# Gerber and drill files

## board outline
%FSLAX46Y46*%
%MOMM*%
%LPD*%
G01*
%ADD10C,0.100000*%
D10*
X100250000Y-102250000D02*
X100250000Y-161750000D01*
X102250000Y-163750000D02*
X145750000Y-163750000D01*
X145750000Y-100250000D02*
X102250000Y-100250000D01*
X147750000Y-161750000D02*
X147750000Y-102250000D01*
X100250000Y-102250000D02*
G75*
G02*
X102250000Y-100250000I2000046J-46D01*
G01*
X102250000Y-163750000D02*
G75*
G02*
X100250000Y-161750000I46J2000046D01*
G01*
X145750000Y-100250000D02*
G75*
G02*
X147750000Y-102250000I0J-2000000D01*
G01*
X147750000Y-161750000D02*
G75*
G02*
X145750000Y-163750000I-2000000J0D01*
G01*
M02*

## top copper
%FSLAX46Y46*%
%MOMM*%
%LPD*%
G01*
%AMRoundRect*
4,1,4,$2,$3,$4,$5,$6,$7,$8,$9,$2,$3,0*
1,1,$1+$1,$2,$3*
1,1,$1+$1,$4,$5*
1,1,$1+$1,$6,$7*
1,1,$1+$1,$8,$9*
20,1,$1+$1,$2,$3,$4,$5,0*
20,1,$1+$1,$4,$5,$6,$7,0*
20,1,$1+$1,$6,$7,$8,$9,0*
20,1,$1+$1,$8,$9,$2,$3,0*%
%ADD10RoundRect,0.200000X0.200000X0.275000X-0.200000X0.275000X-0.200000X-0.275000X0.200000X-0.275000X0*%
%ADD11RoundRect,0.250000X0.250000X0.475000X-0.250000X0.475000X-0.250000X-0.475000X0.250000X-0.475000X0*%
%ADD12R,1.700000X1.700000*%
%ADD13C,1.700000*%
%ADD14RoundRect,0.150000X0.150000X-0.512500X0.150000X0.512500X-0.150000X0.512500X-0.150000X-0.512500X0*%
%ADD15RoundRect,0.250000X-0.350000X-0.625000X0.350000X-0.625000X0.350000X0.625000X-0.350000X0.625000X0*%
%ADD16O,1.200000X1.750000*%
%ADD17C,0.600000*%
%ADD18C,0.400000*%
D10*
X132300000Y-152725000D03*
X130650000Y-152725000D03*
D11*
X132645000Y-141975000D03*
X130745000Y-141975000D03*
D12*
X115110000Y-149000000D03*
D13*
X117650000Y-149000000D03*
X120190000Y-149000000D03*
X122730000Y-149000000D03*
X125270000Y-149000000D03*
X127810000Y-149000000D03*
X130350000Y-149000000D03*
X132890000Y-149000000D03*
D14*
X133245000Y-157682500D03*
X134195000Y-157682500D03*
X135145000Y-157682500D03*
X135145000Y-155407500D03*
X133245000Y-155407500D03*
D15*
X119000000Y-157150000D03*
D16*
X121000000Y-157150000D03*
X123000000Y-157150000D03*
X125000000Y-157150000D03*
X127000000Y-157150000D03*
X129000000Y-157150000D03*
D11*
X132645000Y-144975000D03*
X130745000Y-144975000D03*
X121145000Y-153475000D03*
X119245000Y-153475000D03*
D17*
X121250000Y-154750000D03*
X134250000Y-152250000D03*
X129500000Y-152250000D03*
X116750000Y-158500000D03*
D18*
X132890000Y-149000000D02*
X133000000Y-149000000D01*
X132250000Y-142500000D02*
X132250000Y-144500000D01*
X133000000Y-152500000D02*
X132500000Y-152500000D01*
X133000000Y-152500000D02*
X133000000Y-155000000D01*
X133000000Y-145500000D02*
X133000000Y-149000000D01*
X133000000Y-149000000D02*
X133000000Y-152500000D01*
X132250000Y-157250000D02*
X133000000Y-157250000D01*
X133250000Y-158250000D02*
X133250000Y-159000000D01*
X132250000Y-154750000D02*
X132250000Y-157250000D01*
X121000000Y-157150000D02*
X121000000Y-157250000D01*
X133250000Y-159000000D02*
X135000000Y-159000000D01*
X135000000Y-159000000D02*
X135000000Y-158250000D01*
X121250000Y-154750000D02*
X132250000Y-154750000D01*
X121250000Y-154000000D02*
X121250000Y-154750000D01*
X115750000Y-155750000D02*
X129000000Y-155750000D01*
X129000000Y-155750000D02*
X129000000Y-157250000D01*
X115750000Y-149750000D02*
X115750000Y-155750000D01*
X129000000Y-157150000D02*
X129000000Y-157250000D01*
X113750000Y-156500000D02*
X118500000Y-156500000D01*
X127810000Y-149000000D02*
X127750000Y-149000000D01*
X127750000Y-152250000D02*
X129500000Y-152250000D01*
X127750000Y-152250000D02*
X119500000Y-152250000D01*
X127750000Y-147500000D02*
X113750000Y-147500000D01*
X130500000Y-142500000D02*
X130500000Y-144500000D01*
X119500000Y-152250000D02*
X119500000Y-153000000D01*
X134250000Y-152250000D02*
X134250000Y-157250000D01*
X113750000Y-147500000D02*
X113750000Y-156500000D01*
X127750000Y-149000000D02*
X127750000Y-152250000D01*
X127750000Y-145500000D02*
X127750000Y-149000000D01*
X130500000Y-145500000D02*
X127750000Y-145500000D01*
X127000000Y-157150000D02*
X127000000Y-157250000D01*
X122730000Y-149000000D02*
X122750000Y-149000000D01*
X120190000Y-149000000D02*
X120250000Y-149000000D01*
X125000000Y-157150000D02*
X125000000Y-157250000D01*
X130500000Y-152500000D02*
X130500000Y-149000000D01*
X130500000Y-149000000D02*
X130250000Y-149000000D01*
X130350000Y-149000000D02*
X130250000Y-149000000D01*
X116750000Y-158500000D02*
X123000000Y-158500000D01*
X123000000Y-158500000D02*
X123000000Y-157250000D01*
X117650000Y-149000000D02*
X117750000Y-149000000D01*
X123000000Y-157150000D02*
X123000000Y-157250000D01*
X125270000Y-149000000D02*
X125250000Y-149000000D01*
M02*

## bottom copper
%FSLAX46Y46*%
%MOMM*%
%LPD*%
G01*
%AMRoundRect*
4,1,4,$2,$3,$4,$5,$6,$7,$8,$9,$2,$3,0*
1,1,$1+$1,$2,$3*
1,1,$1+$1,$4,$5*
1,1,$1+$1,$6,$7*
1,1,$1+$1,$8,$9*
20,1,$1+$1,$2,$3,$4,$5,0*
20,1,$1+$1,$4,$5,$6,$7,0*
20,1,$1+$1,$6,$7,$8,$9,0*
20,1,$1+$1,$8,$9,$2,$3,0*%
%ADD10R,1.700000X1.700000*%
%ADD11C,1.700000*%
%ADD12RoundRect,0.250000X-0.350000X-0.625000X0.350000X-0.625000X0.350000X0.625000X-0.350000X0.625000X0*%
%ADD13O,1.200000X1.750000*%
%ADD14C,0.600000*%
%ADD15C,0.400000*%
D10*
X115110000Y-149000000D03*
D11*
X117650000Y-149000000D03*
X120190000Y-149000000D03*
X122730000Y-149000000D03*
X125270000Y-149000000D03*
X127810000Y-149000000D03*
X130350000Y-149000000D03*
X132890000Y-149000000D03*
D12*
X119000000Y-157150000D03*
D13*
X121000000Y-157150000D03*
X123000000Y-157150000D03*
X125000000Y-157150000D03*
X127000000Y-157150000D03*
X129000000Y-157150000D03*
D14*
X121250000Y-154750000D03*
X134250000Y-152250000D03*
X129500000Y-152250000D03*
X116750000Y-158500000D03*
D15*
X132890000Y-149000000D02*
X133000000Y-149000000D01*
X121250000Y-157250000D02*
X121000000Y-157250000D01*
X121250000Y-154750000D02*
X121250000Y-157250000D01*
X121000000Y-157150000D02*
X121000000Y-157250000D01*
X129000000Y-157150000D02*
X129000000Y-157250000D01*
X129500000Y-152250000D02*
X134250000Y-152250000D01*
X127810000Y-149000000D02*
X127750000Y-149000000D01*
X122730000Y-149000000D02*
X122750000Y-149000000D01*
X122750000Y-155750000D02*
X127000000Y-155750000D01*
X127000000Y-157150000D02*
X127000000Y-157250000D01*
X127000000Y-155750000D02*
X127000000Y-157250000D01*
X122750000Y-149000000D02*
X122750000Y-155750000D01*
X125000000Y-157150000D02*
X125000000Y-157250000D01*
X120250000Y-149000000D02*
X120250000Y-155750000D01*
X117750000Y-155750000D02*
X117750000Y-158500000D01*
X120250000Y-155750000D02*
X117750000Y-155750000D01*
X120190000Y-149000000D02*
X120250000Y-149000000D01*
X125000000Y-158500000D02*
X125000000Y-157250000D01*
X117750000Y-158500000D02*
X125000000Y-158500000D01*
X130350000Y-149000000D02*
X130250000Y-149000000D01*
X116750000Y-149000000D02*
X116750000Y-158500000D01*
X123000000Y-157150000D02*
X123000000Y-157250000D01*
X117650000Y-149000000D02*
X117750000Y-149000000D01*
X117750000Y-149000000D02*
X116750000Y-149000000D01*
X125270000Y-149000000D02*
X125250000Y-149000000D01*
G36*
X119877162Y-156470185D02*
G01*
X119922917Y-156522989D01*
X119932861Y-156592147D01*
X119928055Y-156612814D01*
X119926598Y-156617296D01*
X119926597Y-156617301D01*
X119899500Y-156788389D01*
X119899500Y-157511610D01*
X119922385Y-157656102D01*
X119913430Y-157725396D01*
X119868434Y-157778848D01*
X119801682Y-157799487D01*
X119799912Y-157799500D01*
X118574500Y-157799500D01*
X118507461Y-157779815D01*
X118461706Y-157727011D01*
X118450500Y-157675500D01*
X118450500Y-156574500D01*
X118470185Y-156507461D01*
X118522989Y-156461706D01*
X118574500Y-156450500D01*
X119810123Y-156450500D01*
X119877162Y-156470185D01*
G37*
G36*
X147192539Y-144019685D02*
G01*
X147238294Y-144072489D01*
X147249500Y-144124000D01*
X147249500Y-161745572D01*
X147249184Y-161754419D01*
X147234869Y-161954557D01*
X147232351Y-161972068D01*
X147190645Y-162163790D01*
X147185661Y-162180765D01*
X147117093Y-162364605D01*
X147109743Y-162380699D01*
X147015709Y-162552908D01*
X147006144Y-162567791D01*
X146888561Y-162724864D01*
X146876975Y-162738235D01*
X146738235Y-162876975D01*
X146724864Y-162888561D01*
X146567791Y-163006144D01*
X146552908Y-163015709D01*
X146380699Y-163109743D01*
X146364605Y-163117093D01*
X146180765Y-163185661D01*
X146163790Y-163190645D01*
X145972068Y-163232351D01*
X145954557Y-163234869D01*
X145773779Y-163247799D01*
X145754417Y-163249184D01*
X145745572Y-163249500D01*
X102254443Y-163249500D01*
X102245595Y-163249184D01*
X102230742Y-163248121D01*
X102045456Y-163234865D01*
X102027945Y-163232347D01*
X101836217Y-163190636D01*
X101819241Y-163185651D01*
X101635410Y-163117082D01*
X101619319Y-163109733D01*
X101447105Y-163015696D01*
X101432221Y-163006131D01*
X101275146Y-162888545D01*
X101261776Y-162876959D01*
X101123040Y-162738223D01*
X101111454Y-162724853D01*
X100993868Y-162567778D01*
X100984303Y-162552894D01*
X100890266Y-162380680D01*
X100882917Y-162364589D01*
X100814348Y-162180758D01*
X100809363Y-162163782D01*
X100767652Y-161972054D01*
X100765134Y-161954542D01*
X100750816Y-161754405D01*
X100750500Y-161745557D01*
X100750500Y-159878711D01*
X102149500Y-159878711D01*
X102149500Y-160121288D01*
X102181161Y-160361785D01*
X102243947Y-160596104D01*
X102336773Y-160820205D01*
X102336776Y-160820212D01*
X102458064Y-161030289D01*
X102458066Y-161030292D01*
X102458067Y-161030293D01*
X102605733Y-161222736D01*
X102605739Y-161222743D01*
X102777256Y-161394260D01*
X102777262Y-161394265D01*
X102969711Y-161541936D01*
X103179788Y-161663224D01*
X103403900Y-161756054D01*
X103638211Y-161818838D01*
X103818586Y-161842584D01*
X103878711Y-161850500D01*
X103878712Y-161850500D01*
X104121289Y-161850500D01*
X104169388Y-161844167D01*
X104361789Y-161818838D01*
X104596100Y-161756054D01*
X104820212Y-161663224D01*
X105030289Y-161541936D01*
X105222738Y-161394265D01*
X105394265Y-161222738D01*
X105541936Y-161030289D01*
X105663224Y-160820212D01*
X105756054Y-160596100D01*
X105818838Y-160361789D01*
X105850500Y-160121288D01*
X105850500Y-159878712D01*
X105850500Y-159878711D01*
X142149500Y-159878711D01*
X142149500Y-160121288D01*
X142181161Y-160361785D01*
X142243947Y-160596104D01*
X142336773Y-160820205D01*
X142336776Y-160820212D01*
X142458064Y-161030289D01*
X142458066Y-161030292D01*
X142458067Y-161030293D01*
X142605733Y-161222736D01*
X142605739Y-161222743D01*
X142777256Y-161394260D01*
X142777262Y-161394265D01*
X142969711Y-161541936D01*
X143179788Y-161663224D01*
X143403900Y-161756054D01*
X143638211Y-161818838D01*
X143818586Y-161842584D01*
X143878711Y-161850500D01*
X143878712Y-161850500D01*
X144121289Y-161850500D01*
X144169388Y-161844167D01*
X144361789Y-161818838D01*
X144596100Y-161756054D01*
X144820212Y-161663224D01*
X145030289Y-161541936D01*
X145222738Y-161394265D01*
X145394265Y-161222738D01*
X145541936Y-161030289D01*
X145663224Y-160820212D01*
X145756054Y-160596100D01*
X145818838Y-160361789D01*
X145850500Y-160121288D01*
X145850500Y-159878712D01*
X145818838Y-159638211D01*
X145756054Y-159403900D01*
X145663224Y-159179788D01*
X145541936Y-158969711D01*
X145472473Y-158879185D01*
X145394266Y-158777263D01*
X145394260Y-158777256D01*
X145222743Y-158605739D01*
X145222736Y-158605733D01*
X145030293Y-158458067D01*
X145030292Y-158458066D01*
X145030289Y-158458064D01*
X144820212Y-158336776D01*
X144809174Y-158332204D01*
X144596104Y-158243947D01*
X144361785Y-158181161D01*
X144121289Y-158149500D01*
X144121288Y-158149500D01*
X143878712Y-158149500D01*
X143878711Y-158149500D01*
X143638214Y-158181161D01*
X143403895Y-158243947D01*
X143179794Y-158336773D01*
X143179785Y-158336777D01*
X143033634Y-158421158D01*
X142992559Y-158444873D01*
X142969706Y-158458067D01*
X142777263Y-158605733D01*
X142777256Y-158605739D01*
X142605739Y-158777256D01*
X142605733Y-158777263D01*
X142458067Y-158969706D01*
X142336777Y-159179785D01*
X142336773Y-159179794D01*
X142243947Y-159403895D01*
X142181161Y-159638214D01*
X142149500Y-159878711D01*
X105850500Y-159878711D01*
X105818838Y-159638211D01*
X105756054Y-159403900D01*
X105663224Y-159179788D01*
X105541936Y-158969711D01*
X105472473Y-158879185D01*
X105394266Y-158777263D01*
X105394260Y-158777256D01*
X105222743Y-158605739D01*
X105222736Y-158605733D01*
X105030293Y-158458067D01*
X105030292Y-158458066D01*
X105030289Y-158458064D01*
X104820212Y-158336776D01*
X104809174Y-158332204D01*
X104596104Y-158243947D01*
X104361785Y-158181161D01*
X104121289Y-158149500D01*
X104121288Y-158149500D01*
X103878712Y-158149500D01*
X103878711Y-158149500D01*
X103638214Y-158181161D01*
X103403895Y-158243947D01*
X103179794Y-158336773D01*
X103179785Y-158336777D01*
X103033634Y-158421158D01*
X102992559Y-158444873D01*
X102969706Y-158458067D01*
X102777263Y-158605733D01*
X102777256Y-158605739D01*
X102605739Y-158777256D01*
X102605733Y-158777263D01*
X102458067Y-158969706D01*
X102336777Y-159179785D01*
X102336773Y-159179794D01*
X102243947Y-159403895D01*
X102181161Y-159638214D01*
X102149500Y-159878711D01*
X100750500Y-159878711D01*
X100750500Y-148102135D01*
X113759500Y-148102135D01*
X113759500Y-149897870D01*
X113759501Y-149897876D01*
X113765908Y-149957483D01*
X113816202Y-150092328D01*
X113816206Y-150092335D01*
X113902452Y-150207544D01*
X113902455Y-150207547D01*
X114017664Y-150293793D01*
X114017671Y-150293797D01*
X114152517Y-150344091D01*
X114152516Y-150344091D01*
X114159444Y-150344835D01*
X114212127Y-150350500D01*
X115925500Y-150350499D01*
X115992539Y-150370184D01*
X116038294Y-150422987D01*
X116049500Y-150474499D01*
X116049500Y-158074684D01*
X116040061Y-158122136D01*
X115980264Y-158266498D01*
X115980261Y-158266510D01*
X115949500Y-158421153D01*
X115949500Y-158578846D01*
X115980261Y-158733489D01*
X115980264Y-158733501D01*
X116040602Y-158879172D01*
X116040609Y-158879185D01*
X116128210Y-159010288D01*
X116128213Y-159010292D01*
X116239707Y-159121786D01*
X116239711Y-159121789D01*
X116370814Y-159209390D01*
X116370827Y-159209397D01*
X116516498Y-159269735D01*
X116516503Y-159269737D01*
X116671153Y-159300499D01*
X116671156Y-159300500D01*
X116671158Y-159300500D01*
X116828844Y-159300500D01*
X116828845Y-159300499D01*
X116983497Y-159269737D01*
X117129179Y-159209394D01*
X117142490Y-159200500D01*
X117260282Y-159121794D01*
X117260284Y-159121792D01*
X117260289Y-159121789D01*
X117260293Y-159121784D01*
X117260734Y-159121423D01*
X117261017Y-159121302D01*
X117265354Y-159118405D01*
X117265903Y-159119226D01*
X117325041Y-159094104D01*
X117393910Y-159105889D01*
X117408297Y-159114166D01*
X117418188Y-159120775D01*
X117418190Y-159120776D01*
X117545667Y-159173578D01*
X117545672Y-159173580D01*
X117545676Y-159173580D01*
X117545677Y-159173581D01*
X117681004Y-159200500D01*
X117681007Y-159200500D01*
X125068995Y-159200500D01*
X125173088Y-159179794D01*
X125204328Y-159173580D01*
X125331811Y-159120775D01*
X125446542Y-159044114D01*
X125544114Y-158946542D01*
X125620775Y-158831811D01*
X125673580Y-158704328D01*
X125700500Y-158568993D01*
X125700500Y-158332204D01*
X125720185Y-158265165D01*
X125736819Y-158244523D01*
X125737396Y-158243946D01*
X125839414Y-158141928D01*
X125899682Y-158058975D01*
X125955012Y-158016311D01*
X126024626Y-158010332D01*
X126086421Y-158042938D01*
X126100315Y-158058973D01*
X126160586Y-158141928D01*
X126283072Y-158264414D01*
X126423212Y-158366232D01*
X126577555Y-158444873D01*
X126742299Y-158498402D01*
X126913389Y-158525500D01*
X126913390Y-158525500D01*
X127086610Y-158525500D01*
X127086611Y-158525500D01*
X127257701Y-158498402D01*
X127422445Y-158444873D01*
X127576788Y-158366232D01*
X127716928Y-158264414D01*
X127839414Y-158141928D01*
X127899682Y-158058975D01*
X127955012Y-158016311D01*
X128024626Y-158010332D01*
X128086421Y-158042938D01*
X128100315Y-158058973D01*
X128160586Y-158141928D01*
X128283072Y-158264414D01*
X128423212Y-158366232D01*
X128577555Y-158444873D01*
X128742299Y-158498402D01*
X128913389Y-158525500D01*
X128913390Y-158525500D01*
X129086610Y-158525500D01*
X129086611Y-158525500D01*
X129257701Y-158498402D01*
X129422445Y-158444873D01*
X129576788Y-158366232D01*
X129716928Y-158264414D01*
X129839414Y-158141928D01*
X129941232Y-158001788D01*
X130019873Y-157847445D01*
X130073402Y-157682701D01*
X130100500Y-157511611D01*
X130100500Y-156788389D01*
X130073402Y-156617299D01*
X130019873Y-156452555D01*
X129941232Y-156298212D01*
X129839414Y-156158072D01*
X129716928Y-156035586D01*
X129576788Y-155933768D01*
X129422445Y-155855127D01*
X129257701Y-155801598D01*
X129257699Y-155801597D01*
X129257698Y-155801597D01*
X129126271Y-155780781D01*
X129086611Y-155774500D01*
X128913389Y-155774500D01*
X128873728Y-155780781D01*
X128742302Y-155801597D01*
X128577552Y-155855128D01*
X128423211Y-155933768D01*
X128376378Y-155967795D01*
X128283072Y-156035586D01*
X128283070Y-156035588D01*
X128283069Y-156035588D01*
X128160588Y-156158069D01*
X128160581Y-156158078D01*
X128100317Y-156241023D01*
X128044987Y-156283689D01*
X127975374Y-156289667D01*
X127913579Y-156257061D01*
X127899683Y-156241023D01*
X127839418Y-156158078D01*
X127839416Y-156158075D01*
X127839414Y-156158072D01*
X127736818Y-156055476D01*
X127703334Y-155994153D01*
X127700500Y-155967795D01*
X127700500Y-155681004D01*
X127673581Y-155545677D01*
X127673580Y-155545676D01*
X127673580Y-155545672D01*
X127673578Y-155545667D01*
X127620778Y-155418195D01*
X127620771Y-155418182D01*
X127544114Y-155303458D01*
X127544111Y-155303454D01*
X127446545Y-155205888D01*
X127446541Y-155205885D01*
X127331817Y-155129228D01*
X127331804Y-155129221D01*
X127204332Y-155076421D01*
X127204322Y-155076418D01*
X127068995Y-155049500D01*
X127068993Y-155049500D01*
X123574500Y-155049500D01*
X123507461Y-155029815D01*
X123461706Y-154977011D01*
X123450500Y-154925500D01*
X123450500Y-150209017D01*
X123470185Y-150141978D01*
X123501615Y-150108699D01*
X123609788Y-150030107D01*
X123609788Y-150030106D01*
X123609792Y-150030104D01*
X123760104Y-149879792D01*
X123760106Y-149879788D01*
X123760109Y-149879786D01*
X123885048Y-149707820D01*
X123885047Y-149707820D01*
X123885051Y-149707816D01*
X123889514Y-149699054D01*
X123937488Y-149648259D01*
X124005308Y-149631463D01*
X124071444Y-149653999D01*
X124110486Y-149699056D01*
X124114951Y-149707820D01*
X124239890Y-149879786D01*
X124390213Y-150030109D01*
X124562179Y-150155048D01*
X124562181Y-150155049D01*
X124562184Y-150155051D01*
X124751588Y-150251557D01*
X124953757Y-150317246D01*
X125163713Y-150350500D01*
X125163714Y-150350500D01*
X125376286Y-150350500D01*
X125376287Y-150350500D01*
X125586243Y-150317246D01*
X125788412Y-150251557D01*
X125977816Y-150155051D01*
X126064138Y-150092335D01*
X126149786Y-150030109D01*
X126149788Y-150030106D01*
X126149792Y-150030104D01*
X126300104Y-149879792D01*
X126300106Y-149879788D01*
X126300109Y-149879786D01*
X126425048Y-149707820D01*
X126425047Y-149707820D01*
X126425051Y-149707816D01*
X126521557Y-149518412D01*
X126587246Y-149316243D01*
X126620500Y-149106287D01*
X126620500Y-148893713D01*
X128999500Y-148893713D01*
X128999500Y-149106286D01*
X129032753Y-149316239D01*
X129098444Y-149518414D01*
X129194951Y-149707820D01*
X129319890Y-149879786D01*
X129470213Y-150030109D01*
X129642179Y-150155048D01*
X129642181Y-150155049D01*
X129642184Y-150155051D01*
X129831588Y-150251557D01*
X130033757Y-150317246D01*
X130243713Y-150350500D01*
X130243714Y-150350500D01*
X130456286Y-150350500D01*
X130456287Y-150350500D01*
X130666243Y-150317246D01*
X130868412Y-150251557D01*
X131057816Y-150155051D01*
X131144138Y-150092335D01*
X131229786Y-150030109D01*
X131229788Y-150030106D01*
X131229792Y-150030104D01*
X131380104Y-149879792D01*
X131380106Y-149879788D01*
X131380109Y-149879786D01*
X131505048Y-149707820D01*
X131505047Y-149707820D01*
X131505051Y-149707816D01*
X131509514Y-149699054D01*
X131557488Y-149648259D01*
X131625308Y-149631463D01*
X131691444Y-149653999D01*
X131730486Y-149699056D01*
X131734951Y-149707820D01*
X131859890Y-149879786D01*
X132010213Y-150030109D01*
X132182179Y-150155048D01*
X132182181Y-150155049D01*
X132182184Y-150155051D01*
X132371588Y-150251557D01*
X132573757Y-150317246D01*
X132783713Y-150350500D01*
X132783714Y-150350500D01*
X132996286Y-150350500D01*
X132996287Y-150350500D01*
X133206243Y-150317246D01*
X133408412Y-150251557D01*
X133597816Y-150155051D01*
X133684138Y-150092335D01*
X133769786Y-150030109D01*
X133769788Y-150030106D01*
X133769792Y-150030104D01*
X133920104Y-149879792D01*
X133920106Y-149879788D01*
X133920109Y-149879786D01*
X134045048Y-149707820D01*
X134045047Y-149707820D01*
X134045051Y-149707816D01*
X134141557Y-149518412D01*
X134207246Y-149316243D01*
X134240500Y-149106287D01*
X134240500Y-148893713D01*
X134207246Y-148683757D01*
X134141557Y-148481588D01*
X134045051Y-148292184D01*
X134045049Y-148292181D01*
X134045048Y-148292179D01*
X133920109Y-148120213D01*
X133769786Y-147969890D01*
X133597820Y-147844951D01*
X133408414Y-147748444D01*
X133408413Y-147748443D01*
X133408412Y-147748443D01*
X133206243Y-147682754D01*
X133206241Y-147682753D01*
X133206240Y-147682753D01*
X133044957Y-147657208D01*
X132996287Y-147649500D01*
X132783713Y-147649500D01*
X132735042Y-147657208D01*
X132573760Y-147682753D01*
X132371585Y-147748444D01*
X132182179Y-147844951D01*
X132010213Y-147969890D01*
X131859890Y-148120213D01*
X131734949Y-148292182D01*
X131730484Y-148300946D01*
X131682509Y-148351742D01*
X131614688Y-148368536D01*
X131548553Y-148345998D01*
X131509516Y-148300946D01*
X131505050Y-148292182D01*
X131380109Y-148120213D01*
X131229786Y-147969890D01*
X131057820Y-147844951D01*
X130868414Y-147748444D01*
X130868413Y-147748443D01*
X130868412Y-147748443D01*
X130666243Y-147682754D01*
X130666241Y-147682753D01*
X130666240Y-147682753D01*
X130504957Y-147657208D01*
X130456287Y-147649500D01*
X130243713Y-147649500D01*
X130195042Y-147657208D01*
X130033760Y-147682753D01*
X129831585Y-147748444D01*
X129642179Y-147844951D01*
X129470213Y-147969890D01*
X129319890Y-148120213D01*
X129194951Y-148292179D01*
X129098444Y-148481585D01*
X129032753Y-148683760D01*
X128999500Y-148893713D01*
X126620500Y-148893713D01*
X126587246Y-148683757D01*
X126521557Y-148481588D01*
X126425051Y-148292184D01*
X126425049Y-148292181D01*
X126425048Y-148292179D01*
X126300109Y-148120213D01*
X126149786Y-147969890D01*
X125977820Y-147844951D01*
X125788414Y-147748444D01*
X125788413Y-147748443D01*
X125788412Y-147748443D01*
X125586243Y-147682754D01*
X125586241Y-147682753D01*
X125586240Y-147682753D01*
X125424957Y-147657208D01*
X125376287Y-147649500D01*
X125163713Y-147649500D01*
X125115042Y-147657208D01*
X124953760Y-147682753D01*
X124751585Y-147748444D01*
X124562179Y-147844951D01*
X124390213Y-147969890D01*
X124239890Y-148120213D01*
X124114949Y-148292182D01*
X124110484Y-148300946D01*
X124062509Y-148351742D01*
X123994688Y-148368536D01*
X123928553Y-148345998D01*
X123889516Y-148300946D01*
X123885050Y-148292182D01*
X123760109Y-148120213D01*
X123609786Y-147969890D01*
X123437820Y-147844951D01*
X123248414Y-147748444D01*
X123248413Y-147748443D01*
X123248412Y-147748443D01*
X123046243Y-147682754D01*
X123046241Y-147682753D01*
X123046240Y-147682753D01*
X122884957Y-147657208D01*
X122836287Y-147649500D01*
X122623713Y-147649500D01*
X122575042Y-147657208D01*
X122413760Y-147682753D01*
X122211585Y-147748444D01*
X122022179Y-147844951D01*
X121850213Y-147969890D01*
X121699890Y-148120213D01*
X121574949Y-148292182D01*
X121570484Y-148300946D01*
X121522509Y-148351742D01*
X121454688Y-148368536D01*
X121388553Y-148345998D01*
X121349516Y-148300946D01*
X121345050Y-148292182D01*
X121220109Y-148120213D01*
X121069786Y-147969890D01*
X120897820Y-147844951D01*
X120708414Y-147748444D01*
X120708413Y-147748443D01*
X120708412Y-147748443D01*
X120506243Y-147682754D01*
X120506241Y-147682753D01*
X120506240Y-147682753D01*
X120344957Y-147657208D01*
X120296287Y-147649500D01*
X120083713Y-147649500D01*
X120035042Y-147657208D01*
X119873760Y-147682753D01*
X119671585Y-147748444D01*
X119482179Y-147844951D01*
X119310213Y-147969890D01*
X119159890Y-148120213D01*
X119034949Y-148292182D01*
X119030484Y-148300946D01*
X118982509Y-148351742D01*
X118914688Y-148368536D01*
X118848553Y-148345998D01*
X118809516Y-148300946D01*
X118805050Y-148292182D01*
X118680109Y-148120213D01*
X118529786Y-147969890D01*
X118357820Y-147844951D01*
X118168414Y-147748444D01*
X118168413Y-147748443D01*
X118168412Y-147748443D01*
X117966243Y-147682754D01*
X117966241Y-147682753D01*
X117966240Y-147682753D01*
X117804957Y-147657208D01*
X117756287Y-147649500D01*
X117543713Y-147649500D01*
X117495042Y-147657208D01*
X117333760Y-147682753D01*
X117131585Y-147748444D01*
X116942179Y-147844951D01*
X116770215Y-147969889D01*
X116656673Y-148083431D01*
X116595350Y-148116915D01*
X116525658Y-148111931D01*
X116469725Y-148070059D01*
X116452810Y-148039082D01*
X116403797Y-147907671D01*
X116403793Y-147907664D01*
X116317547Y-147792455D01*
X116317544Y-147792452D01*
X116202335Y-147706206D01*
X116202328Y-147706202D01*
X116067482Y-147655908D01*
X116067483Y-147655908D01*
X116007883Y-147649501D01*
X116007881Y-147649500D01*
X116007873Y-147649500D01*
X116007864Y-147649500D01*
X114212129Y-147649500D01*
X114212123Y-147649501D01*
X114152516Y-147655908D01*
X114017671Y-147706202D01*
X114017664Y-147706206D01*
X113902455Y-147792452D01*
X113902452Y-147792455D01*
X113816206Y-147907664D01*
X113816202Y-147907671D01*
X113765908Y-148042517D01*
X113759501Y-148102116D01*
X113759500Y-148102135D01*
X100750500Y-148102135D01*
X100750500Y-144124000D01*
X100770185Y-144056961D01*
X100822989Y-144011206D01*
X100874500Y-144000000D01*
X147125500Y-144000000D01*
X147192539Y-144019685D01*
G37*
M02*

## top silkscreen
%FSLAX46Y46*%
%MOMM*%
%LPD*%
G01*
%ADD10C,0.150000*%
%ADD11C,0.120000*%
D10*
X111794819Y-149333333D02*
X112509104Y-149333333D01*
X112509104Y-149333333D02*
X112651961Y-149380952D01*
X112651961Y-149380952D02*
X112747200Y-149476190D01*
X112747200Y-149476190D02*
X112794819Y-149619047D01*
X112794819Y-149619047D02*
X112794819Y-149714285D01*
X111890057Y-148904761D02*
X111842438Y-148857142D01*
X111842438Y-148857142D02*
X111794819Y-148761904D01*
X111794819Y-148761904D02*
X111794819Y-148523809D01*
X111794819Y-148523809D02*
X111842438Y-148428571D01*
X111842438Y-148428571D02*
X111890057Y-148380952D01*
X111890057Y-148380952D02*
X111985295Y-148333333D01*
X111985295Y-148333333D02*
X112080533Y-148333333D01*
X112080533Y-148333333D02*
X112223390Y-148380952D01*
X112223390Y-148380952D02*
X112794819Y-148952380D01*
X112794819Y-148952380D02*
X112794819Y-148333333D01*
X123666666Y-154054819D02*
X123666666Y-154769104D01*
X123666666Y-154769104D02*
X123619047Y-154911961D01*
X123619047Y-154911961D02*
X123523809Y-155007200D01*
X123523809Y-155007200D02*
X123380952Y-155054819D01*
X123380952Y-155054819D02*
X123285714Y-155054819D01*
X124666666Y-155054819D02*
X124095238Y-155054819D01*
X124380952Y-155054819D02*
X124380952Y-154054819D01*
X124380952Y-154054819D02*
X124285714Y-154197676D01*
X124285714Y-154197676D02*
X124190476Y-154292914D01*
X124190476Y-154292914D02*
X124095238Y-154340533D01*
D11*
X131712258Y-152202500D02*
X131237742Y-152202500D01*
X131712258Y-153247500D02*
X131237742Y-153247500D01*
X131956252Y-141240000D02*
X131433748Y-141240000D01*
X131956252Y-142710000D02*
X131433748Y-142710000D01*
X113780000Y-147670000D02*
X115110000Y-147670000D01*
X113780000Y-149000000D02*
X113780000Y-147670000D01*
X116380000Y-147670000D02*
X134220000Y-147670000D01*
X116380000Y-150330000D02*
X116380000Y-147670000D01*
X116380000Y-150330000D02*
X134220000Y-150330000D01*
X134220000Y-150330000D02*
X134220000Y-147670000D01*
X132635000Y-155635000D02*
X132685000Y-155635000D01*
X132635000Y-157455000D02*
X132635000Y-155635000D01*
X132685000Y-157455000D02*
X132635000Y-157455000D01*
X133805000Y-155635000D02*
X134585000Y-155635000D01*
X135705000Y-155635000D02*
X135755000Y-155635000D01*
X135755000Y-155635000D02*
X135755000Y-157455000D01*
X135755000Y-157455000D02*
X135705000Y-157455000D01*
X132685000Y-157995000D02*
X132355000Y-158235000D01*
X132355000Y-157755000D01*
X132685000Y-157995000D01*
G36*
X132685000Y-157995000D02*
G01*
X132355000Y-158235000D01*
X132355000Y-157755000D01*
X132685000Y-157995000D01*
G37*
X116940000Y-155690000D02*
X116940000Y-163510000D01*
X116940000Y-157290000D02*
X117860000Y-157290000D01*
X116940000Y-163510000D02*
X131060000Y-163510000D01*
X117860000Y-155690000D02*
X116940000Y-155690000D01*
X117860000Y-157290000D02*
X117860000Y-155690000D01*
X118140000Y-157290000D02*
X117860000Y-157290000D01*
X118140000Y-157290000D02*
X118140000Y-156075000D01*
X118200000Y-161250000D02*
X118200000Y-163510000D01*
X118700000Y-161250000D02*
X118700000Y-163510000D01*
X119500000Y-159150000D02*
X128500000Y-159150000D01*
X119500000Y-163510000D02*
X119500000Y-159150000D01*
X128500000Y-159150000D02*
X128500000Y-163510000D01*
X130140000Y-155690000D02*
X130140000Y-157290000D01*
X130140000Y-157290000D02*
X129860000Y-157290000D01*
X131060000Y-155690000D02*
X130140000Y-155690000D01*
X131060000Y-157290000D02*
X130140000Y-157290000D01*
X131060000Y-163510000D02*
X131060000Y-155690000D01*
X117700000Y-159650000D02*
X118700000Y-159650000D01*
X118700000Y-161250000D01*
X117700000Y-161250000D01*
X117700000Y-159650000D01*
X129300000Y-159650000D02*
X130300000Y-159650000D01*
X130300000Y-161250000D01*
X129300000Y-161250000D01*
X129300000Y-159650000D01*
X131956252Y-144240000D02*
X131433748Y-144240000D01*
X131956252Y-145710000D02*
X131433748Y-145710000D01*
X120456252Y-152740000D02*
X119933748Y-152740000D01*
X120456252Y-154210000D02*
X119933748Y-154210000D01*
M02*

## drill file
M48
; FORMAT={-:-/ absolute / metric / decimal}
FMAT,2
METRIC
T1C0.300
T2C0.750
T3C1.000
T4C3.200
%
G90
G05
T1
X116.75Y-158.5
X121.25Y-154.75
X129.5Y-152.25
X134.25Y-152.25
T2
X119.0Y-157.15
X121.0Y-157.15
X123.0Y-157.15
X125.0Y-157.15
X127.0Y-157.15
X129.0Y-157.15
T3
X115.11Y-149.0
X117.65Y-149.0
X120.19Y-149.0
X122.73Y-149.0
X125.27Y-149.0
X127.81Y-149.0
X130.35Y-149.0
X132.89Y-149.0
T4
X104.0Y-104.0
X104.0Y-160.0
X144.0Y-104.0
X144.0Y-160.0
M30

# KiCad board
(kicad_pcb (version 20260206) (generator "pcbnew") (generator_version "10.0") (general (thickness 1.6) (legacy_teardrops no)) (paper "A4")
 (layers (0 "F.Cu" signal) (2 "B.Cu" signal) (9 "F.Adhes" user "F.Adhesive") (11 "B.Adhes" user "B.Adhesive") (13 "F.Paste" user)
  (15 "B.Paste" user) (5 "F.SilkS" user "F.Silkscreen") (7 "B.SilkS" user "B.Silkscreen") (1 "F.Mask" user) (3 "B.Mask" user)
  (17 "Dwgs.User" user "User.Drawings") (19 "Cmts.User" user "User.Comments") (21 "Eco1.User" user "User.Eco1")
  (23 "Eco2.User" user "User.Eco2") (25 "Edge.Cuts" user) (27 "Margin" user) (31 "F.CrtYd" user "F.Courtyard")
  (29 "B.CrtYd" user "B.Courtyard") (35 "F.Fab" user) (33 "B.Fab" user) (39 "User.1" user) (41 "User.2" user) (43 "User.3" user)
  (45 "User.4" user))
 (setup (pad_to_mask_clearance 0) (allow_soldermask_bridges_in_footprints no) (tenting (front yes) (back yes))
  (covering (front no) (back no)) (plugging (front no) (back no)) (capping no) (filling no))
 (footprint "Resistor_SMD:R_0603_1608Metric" (layer "F.Cu") (at 131.475 152.725 180)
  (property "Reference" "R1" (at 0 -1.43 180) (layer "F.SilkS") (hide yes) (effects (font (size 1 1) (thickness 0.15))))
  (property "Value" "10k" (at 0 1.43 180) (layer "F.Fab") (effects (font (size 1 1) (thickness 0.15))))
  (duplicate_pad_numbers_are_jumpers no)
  (fp_line (start -0.237258 0.5225) (end 0.237258 0.5225) (stroke (width 0.12) (type solid)) (layer "F.SilkS"))
  (fp_line (start -0.237258 -0.5225) (end 0.237258 -0.5225) (stroke (width 0.12) (type solid)) (layer "F.SilkS"))
  (pad "1" smd roundrect (at -0.825 0 180) (size 0.8 0.95) (layers "F.Cu" "F.Mask" "F.Paste") (roundrect_rratio 0.25) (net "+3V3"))
  (pad "2" smd roundrect (at 0.825 0 180) (size 0.8 0.95) (layers "F.Cu" "F.Mask" "F.Paste") (roundrect_rratio 0.25) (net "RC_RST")))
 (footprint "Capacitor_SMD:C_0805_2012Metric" (layer "F.Cu") (at 131.695 141.975 180)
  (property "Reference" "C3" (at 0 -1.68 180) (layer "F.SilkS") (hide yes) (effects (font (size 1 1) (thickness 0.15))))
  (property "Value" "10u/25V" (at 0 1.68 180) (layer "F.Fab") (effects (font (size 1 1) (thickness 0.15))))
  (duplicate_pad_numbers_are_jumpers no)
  (fp_line (start -0.261252 0.735) (end 0.261252 0.735) (stroke (width 0.12) (type solid)) (layer "F.SilkS"))
  (fp_line (start -0.261252 -0.735) (end 0.261252 -0.735) (stroke (width 0.12) (type solid)) (layer "F.SilkS"))
  (pad "1" smd roundrect (at -0.95 0 180) (size 1 1.45) (layers "F.Cu" "F.Mask" "F.Paste") (roundrect_rratio 0.25) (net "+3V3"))
  (pad "2" smd roundrect (at 0.95 0 180) (size 1 1.45) (layers "F.Cu" "F.Mask" "F.Paste") (roundrect_rratio 0.25) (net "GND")))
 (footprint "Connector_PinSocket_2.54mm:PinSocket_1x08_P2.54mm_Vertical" (layer "F.Cu") (at 115.11 149 90)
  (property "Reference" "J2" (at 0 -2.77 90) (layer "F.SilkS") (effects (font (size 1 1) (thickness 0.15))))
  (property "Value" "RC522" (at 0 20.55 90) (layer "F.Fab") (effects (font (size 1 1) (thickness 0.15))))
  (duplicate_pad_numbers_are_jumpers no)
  (fp_line (start 1.33 -1.33) (end 1.33 0) (stroke (width 0.12) (type solid)) (layer "F.SilkS"))
  (fp_line (start 0 -1.33) (end 1.33 -1.33) (stroke (width 0.12) (type solid)) (layer "F.SilkS"))
  (fp_line (start 1.33 1.27) (end 1.33 19.11) (stroke (width 0.12) (type solid)) (layer "F.SilkS"))
  (fp_line (start -1.33 1.27) (end 1.33 1.27) (stroke (width 0.12) (type solid)) (layer "F.SilkS"))
  (fp_line (start -1.33 1.27) (end -1.33 19.11) (stroke (width 0.12) (type solid)) (layer "F.SilkS"))
  (fp_line (start -1.33 19.11) (end 1.33 19.11) (stroke (width 0.12) (type solid)) (layer "F.SilkS"))
  (pad "1" thru_hole rect (at 0 0 90) (size 1.7 1.7) (drill 1) (layers "*.Cu" "*.Mask") (remove_unused_layers no) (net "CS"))
  (pad "2" thru_hole circle (at 0 2.54 90) (size 1.7 1.7) (drill 1) (layers "*.Cu" "*.Mask") (remove_unused_layers no) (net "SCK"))
  (pad "3" thru_hole circle (at 0 5.08 90) (size 1.7 1.7) (drill 1) (layers "*.Cu" "*.Mask") (remove_unused_layers no) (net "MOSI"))
  (pad "4" thru_hole circle (at 0 7.62 90) (size 1.7 1.7) (drill 1) (layers "*.Cu" "*.Mask") (remove_unused_layers no) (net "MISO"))
  (pad "5" thru_hole circle (at 0 10.16 90) (size 1.7 1.7) (drill 1) (layers "*.Cu" "*.Mask") (remove_unused_layers no)
   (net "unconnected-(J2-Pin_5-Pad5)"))
  (pad "6" thru_hole circle (at 0 12.7 90) (size 1.7 1.7) (drill 1) (layers "*.Cu" "*.Mask") (remove_unused_layers no) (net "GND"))
  (pad "7" thru_hole circle (at 0 15.24 90) (size 1.7 1.7) (drill 1) (layers "*.Cu" "*.Mask") (remove_unused_layers no) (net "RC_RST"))
  (pad "8" thru_hole circle (at 0 17.78 90) (size 1.7 1.7) (drill 1) (layers "*.Cu" "*.Mask") (remove_unused_layers no) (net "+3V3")))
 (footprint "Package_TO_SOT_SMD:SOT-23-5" (layer "F.Cu") (at 134.195 156.545 90)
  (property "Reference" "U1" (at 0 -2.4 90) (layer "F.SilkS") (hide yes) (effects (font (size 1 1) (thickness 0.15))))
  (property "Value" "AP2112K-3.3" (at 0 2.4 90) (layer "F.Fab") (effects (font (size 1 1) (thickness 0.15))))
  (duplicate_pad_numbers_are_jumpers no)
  (fp_line (start 0.91 -1.56) (end 0.91 -1.51) (stroke (width 0.12) (type solid)) (layer "F.SilkS"))
  (fp_line (start -0.91 -1.56) (end 0.91 -1.56) (stroke (width 0.12) (type solid)) (layer "F.SilkS"))
  (fp_line (start -0.91 -1.51) (end -0.91 -1.56) (stroke (width 0.12) (type solid)) (layer "F.SilkS"))
  (fp_line (start 0.91 -0.39) (end 0.91 0.39) (stroke (width 0.12) (type solid)) (layer "F.SilkS"))
  (fp_line (start 0.91 1.51) (end 0.91 1.56) (stroke (width 0.12) (type solid)) (layer "F.SilkS"))
  (fp_line (start 0.91 1.56) (end -0.91 1.56) (stroke (width 0.12) (type solid)) (layer "F.SilkS"))
  (fp_line (start -0.91 1.56) (end -0.91 1.51) (stroke (width 0.12) (type solid)) (layer "F.SilkS"))
  (fp_poly (pts (xy -1.45 -1.51) (xy -1.69 -1.84) (xy -1.21 -1.84)) (stroke (width 0.12) (type solid)) (fill yes) (layer "F.SilkS"))
  (pad "1" smd roundrect (at -1.1375 -0.95 90) (size 1.325 0.6) (layers "F.Cu" "F.Mask" "F.Paste") (roundrect_rratio 0.25) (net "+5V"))
  (pad "2" smd roundrect (at -1.1375 0 90) (size 1.325 0.6) (layers "F.Cu" "F.Mask" "F.Paste") (roundrect_rratio 0.25) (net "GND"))
  (pad "3" smd roundrect (at -1.1375 0.95 90) (size 1.325 0.6) (layers "F.Cu" "F.Mask" "F.Paste") (roundrect_rratio 0.25) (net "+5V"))
  (pad "4" smd roundrect (at 1.1375 0.95 90) (size 1.325 0.6) (layers "F.Cu" "F.Mask" "F.Paste") (roundrect_rratio 0.25)
   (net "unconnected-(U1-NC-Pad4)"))
  (pad "5" smd roundrect (at 1.1375 -0.95 90) (size 1.325 0.6) (layers "F.Cu" "F.Mask" "F.Paste") (roundrect_rratio 0.25) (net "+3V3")))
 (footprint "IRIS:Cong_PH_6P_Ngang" (layer "F.Cu") (at 119 157.15)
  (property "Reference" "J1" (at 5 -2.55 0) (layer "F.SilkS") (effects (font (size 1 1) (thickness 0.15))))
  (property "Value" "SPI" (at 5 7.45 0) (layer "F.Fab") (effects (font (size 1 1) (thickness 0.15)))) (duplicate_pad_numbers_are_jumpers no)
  (fp_line (start -2.06 -1.46) (end -2.06 6.36) (stroke (width 0.12) (type solid)) (layer "F.SilkS"))
  (fp_line (start -2.06 0.14) (end -1.14 0.14) (stroke (width 0.12) (type solid)) (layer "F.SilkS"))
  (fp_line (start -2.06 6.36) (end 12.06 6.36) (stroke (width 0.12) (type solid)) (layer "F.SilkS"))
  (fp_line (start -1.14 -1.46) (end -2.06 -1.46) (stroke (width 0.12) (type solid)) (layer "F.SilkS"))
  (fp_line (start -1.14 0.14) (end -1.14 -1.46) (stroke (width 0.12) (type solid)) (layer "F.SilkS"))
  (fp_line (start -0.86 0.14) (end -1.14 0.14) (stroke (width 0.12) (type solid)) (layer "F.SilkS"))
  (fp_line (start -0.86 0.14) (end -0.86 -1.075) (stroke (width 0.12) (type solid)) (layer "F.SilkS"))
  (fp_line (start -0.8 4.1) (end -0.8 6.36) (stroke (width 0.12) (type solid)) (layer "F.SilkS"))
  (fp_line (start -0.3 4.1) (end -0.3 6.36) (stroke (width 0.12) (type solid)) (layer "F.SilkS"))
  (fp_line (start 0.5 2) (end 9.5 2) (stroke (width 0.12) (type solid)) (layer "F.SilkS"))
  (fp_line (start 0.5 6.36) (end 0.5 2) (stroke (width 0.12) (type solid)) (layer "F.SilkS"))
  (fp_line (start 9.5 2) (end 9.5 6.36) (stroke (width 0.12) (type solid)) (layer "F.SilkS"))
  (fp_line (start 11.14 -1.46) (end 11.14 0.14) (stroke (width 0.12) (type solid)) (layer "F.SilkS"))
  (fp_line (start 11.14 0.14) (end 10.86 0.14) (stroke (width 0.12) (type solid)) (layer "F.SilkS"))
  (fp_line (start 12.06 -1.46) (end 11.14 -1.46) (stroke (width 0.12) (type solid)) (layer "F.SilkS"))
  (fp_line (start 12.06 0.14) (end 11.14 0.14) (stroke (width 0.12) (type solid)) (layer "F.SilkS"))
  (fp_line (start 12.06 6.36) (end 12.06 -1.46) (stroke (width 0.12) (type solid)) (layer "F.SilkS"))
  (fp_rect (start -1.3 2.5) (end -0.3 4.1) (stroke (width 0.12) (type solid)) (fill no) (layer "F.SilkS"))
  (fp_rect (start 10.3 2.5) (end 11.3 4.1) (stroke (width 0.12) (type solid)) (fill no) (layer "F.SilkS"))
  (pad "1" thru_hole roundrect (at 0 0) (size 1.2 1.75) (drill 0.75) (layers "*.Cu" "*.Mask") (remove_unused_layers no)
   (roundrect_rratio 0.208333) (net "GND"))
  (pad "2" thru_hole oval (at 2 0) (size 1.2 1.75) (drill 0.75) (layers "*.Cu" "*.Mask") (remove_unused_layers no) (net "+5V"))
  (pad "3" thru_hole oval (at 4 0) (size 1.2 1.75) (drill 0.75) (layers "*.Cu" "*.Mask") (remove_unused_layers no) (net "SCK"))
  (pad "4" thru_hole oval (at 6 0) (size 1.2 1.75) (drill 0.75) (layers "*.Cu" "*.Mask") (remove_unused_layers no) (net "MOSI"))
  (pad "5" thru_hole oval (at 8 0) (size 1.2 1.75) (drill 0.75) (layers "*.Cu" "*.Mask") (remove_unused_layers no) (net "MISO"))
  (pad "6" thru_hole oval (at 10 0) (size 1.2 1.75) (drill 0.75) (layers "*.Cu" "*.Mask") (remove_unused_layers no) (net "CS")))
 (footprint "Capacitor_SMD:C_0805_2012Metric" (layer "F.Cu") (at 131.695 144.975 180)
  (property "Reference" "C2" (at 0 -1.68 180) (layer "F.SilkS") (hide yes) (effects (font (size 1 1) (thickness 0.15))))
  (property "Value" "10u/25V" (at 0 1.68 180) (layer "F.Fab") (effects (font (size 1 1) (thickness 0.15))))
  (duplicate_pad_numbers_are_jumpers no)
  (fp_line (start -0.261252 0.735) (end 0.261252 0.735) (stroke (width 0.12) (type solid)) (layer "F.SilkS"))
  (fp_line (start -0.261252 -0.735) (end 0.261252 -0.735) (stroke (width 0.12) (type solid)) (layer "F.SilkS"))
  (pad "1" smd roundrect (at -0.95 0 180) (size 1 1.45) (layers "F.Cu" "F.Mask" "F.Paste") (roundrect_rratio 0.25) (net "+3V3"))
  (pad "2" smd roundrect (at 0.95 0 180) (size 1 1.45) (layers "F.Cu" "F.Mask" "F.Paste") (roundrect_rratio 0.25) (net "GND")))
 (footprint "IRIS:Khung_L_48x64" (layer "F.Cu") (at 100 164)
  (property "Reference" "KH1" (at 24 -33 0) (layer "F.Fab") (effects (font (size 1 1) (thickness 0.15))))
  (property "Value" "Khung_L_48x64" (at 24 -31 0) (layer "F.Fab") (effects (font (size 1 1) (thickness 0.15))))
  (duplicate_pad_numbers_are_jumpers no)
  (fp_line (start 0.25 -61.75) (end 0.25 -2.25) (stroke (width 0.1) (type solid)) (layer "Edge.Cuts"))
  (fp_line (start 2.25 -0.25) (end 45.75 -0.25) (stroke (width 0.1) (type solid)) (layer "Edge.Cuts"))
  (fp_line (start 45.75 -63.75) (end 2.25 -63.75) (stroke (width 0.1) (type solid)) (layer "Edge.Cuts"))
  (fp_line (start 47.75 -2.25) (end 47.75 -61.75) (stroke (width 0.1) (type solid)) (layer "Edge.Cuts"))
  (fp_arc (start 0.25 -61.75) (mid 0.8358 -63.1642) (end 2.25 -63.75) (stroke (width 0.1) (type solid)) (layer "Edge.Cuts"))
  (fp_arc (start 2.25 -0.25) (mid 0.8358 -0.8358) (end 0.25 -2.25) (stroke (width 0.1) (type solid)) (layer "Edge.Cuts"))
  (fp_arc (start 45.75 -63.75) (mid 47.164199 -63.164199) (end 47.75 -61.75) (stroke (width 0.1) (type solid)) (layer "Edge.Cuts"))
  (fp_arc (start 47.75 -2.25) (mid 47.164214 -0.835786) (end 45.75 -0.25) (stroke (width 0.1) (type solid)) (layer "Edge.Cuts"))
  (pad "" np_thru_hole circle (at 4 -60) (size 3.2 3.2) (drill 3.2) (layers "*.Cu" "*.Mask"))
  (pad "" np_thru_hole circle (at 4 -4) (size 3.2 3.2) (drill 3.2) (layers "*.Cu" "*.Mask"))
  (pad "" np_thru_hole circle (at 44 -60) (size 3.2 3.2) (drill 3.2) (layers "*.Cu" "*.Mask"))
  (pad "" np_thru_hole circle (at 44 -4) (size 3.2 3.2) (drill 3.2) (layers "*.Cu" "*.Mask")))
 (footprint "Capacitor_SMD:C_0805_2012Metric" (layer "F.Cu") (at 120.195 153.475 180)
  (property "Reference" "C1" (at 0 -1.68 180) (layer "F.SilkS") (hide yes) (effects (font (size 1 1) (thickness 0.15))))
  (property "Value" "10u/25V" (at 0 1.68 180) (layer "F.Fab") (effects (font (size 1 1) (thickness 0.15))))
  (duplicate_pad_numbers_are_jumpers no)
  (fp_line (start -0.261252 0.735) (end 0.261252 0.735) (stroke (width 0.12) (type solid)) (layer "F.SilkS"))
  (fp_line (start -0.261252 -0.735) (end 0.261252 -0.735) (stroke (width 0.12) (type solid)) (layer "F.SilkS"))
  (pad "1" smd roundrect (at -0.95 0 180) (size 1 1.45) (layers "F.Cu" "F.Mask" "F.Paste") (roundrect_rratio 0.25) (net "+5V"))
  (pad "2" smd roundrect (at 0.95 0 180) (size 1 1.45) (layers "F.Cu" "F.Mask" "F.Paste") (roundrect_rratio 0.25) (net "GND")))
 (segment (start 132.89 149) (end 133 149) (width 0.4) (layer "F.Cu") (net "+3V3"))
 (segment (start 132.25 142.5) (end 132.25 144.5) (width 0.4) (layer "F.Cu") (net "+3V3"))
 (segment (start 133 152.5) (end 132.5 152.5) (width 0.4) (layer "F.Cu") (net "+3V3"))
 (segment (start 133 152.5) (end 133 155) (width 0.4) (layer "F.Cu") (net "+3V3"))
 (segment (start 133 145.5) (end 133 149) (width 0.4) (layer "F.Cu") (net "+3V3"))
 (segment (start 133 149) (end 133 152.5) (width 0.4) (layer "F.Cu") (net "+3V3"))
 (segment (start 132.89 149) (end 133 149) (width 0.4) (layer "B.Cu") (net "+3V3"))
 (segment (start 132.25 157.25) (end 133 157.25) (width 0.4) (layer "F.Cu") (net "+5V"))
 (segment (start 133.25 158.25) (end 133.25 159) (width 0.4) (layer "F.Cu") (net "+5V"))
 (segment (start 132.25 154.75) (end 132.25 157.25) (width 0.4) (layer "F.Cu") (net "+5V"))
 (segment (start 121 157.15) (end 121 157.25) (width 0.4) (layer "F.Cu") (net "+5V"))
 (segment (start 133.25 159) (end 135 159) (width 0.4) (layer "F.Cu") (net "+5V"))
 (segment (start 135 159) (end 135 158.25) (width 0.4) (layer "F.Cu") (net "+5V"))
 (segment (start 121.25 154.75) (end 132.25 154.75) (width 0.4) (layer "F.Cu") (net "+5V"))
 (segment (start 121.25 154) (end 121.25 154.75) (width 0.4) (layer "F.Cu") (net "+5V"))
 (via (at 121.25 154.75) (size 0.6) (drill 0.3) (layers "F.Cu" "B.Cu") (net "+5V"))
 (segment (start 121.25 157.25) (end 121 157.25) (width 0.4) (layer "B.Cu") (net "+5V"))
 (segment (start 121.25 154.75) (end 121.25 157.25) (width 0.4) (layer "B.Cu") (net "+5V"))
 (segment (start 121 157.15) (end 121 157.25) (width 0.4) (layer "B.Cu") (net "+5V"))
 (segment (start 115.75 155.75) (end 129 155.75) (width 0.4) (layer "F.Cu") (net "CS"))
 (segment (start 129 155.75) (end 129 157.25) (width 0.4) (layer "F.Cu") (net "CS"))
 (segment (start 115.75 149.75) (end 115.75 155.75) (width 0.4) (layer "F.Cu") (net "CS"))
 (segment (start 129 157.15) (end 129 157.25) (width 0.4) (layer "F.Cu") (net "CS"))
 (segment (start 129 157.15) (end 129 157.25) (width 0.4) (layer "B.Cu") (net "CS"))
 (segment (start 113.75 156.5) (end 118.5 156.5) (width 0.4) (layer "F.Cu") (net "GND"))
 (segment (start 127.81 149) (end 127.75 149) (width 0.4) (layer "F.Cu") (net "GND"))
 (segment (start 127.75 152.25) (end 129.5 152.25) (width 0.4) (layer "F.Cu") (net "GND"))
 (segment (start 127.75 152.25) (end 119.5 152.25) (width 0.4) (layer "F.Cu") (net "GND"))
 (segment (start 127.75 147.5) (end 113.75 147.5) (width 0.4) (layer "F.Cu") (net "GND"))
 (segment (start 130.5 142.5) (end 130.5 144.5) (width 0.4) (layer "F.Cu") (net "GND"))
 (segment (start 119.5 152.25) (end 119.5 153) (width 0.4) (layer "F.Cu") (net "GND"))
 (segment (start 134.25 152.25) (end 134.25 157.25) (width 0.4) (layer "F.Cu") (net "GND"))
 (segment (start 113.75 147.5) (end 113.75 156.5) (width 0.4) (layer "F.Cu") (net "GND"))
 (segment (start 127.75 149) (end 127.75 152.25) (width 0.4) (layer "F.Cu") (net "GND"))
 (segment (start 127.75 145.5) (end 127.75 149) (width 0.4) (layer "F.Cu") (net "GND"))
 (segment (start 130.5 145.5) (end 127.75 145.5) (width 0.4) (layer "F.Cu") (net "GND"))
 (via (at 134.25 152.25) (size 0.6) (drill 0.3) (layers "F.Cu" "B.Cu") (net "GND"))
 (via (at 129.5 152.25) (size 0.6) (drill 0.3) (layers "F.Cu" "B.Cu") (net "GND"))
 (segment (start 129.5 152.25) (end 134.25 152.25) (width 0.4) (layer "B.Cu") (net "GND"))
 (segment (start 127.81 149) (end 127.75 149) (width 0.4) (layer "B.Cu") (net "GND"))
 (segment (start 127 157.15) (end 127 157.25) (width 0.4) (layer "F.Cu") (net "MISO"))
 (segment (start 122.73 149) (end 122.75 149) (width 0.4) (layer "F.Cu") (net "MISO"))
 (segment (start 122.73 149) (end 122.75 149) (width 0.4) (layer "B.Cu") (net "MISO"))
 (segment (start 122.75 155.75) (end 127 155.75) (width 0.4) (layer "B.Cu") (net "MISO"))
 (segment (start 127 157.15) (end 127 157.25) (width 0.4) (layer "B.Cu") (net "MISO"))
 (segment (start 127 155.75) (end 127 157.25) (width 0.4) (layer "B.Cu") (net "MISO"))
 (segment (start 122.75 149) (end 122.75 155.75) (width 0.4) (layer "B.Cu") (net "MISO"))
 (segment (start 120.19 149) (end 120.25 149) (width 0.4) (layer "F.Cu") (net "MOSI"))
 (segment (start 125 157.15) (end 125 157.25) (width 0.4) (layer "F.Cu") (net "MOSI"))
 (segment (start 125 157.15) (end 125 157.25) (width 0.4) (layer "B.Cu") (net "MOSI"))
 (segment (start 120.25 149) (end 120.25 155.75) (width 0.4) (layer "B.Cu") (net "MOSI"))
 (segment (start 117.75 155.75) (end 117.75 158.5) (width 0.4) (layer "B.Cu") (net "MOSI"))
 (segment (start 120.25 155.75) (end 117.75 155.75) (width 0.4) (layer "B.Cu") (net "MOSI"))
 (segment (start 120.19 149) (end 120.25 149) (width 0.4) (layer "B.Cu") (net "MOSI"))
 (segment (start 125 158.5) (end 125 157.25) (width 0.4) (layer "B.Cu") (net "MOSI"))
 (segment (start 117.75 158.5) (end 125 158.5) (width 0.4) (layer "B.Cu") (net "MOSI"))
 (segment (start 130.5 152.5) (end 130.5 149) (width 0.4) (layer "F.Cu") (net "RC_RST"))
 (segment (start 130.5 149) (end 130.25 149) (width 0.4) (layer "F.Cu") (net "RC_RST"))
 (segment (start 130.35 149) (end 130.25 149) (width 0.4) (layer "F.Cu") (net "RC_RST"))
 (segment (start 130.35 149) (end 130.25 149) (width 0.4) (layer "B.Cu") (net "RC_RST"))
 (segment (start 116.75 158.5) (end 123 158.5) (width 0.4) (layer "F.Cu") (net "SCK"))
 (segment (start 123 158.5) (end 123 157.25) (width 0.4) (layer "F.Cu") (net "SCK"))
 (segment (start 117.65 149) (end 117.75 149) (width 0.4) (layer "F.Cu") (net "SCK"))
 (segment (start 123 157.15) (end 123 157.25) (width 0.4) (layer "F.Cu") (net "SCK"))
 (via (at 116.75 158.5) (size 0.6) (drill 0.3) (layers "F.Cu" "B.Cu") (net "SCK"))
 (segment (start 116.75 149) (end 116.75 158.5) (width 0.4) (layer "B.Cu") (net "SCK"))
 (segment (start 123 157.15) (end 123 157.25) (width 0.4) (layer "B.Cu") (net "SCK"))
 (segment (start 117.65 149) (end 117.75 149) (width 0.4) (layer "B.Cu") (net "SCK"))
 (segment (start 117.75 149) (end 116.75 149) (width 0.4) (layer "B.Cu") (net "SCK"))
 (segment (start 125.27 149) (end 125.25 149) (width 0.4) (layer "F.Cu") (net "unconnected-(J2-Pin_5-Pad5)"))
 (segment (start 125.27 149) (end 125.25 149) (width 0.4) (layer "B.Cu") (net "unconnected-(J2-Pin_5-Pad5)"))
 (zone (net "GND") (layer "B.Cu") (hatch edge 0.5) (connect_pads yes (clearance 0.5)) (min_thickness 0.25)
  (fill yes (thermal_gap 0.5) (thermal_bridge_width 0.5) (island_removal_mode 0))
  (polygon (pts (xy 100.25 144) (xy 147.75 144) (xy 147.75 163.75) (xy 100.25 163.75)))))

